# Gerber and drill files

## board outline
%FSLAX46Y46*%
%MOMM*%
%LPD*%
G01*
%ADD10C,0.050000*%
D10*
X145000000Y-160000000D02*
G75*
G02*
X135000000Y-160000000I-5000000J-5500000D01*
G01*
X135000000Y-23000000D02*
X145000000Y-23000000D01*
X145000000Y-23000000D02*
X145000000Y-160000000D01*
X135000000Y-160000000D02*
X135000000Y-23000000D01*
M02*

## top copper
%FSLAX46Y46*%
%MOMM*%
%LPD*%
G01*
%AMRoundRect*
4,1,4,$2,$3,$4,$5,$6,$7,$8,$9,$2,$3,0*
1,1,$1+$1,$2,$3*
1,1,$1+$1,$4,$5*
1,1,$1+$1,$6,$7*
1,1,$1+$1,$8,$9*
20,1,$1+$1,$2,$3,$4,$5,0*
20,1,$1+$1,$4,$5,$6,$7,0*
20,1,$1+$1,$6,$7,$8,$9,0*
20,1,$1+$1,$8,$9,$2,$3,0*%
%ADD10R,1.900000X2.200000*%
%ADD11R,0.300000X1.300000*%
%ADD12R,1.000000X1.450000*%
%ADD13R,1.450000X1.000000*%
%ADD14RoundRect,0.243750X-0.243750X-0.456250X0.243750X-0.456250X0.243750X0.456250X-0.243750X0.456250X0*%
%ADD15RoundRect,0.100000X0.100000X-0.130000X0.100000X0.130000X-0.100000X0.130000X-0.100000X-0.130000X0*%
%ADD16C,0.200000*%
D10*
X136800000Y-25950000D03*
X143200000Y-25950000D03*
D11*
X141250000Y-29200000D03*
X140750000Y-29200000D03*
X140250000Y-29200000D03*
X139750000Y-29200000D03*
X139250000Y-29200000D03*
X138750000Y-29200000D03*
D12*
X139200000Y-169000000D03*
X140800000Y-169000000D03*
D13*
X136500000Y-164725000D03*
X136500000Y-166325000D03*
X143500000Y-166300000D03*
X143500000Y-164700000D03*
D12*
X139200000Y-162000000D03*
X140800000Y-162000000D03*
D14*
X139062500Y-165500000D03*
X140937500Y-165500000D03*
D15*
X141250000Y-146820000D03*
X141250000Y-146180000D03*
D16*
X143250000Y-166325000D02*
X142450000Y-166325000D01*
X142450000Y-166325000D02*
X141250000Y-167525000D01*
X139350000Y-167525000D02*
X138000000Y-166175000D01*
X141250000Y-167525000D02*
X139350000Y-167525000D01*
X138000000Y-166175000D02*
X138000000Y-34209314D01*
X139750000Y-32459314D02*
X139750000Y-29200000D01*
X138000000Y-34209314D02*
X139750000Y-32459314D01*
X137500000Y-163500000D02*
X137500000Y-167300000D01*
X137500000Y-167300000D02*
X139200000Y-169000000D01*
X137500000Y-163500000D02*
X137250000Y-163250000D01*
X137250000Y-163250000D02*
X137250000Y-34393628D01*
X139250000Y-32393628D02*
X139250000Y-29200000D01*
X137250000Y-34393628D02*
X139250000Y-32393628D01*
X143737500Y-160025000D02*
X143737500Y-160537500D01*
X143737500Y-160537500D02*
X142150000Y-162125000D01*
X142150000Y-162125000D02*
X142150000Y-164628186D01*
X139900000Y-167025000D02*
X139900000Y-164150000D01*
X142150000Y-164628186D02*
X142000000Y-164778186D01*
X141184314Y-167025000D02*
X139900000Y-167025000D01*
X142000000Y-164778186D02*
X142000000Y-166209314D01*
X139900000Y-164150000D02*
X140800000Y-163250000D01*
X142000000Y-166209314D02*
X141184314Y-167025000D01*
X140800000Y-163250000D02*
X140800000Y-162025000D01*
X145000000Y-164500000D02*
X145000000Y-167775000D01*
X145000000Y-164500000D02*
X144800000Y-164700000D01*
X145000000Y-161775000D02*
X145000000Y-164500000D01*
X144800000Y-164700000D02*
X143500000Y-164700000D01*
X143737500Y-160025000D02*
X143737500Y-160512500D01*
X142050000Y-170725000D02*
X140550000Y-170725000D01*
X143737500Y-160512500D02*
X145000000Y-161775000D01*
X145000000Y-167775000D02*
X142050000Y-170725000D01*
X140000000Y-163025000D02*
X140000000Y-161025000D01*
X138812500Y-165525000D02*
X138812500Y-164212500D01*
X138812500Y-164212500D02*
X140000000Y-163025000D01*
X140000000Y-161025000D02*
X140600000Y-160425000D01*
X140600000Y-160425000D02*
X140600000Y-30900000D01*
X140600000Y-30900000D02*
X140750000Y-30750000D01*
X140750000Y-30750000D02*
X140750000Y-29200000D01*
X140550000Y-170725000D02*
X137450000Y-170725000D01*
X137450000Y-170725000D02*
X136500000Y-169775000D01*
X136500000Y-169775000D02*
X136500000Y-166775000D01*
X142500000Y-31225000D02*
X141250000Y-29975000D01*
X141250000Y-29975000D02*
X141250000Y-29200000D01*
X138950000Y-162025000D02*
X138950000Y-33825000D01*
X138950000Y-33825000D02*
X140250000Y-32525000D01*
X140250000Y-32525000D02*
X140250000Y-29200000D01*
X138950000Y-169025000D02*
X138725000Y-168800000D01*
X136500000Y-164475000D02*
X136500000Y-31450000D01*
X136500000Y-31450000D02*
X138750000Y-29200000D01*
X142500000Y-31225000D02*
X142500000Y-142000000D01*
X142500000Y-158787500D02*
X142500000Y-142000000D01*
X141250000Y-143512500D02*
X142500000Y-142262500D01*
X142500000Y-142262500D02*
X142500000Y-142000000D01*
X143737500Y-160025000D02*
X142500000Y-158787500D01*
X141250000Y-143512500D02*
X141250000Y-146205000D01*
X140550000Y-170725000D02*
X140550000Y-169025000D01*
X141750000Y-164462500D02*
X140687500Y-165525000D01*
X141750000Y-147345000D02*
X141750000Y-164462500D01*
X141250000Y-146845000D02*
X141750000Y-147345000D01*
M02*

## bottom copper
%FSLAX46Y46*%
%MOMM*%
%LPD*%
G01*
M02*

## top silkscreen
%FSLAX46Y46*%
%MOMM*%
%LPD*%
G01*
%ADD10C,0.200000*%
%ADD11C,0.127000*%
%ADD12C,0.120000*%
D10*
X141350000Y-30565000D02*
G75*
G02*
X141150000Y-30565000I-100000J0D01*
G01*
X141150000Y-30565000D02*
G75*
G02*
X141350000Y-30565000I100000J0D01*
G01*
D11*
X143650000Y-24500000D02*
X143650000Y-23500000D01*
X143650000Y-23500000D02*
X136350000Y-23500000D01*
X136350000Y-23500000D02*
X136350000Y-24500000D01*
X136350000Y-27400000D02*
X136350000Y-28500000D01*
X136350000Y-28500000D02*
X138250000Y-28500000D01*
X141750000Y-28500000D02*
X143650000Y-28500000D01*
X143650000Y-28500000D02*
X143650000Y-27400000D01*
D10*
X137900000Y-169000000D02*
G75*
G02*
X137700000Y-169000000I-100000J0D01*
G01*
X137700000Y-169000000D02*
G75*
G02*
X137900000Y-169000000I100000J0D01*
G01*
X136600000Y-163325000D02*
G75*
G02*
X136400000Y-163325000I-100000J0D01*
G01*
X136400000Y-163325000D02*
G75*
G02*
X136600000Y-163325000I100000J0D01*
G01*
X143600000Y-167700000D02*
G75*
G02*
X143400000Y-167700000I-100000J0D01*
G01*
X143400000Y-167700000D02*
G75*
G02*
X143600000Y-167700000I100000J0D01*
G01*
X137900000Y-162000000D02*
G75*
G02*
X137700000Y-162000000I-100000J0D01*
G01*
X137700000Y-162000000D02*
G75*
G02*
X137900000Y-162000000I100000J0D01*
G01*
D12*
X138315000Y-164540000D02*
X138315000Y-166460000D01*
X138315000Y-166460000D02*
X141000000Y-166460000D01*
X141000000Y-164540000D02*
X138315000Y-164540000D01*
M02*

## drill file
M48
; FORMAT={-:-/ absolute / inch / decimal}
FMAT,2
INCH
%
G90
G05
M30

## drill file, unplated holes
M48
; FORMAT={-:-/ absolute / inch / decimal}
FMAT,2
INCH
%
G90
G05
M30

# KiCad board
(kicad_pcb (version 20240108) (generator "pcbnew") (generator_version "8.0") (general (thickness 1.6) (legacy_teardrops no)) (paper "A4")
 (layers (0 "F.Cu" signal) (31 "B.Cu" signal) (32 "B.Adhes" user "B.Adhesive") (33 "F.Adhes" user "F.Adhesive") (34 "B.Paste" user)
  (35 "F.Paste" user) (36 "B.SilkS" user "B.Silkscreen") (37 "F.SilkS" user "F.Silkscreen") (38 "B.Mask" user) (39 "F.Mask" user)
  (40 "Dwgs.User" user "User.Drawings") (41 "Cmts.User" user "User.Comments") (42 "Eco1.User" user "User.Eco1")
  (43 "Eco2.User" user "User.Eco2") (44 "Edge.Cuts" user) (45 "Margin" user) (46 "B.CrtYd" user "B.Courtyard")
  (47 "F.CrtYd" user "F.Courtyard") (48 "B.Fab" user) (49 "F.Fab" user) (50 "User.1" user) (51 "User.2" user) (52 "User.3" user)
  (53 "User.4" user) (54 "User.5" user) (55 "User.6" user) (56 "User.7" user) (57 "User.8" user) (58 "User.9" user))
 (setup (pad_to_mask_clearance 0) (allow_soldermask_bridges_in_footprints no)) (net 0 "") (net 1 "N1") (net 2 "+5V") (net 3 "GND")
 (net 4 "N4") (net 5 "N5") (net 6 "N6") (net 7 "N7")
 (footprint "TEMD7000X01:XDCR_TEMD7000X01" (layer "F.Cu") (at 140 169)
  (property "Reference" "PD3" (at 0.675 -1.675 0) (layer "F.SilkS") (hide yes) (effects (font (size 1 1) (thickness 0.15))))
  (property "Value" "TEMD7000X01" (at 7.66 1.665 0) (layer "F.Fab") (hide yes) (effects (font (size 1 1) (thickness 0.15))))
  (fp_circle (center -2.2 0) (end -2.1 0) (stroke (width 0.2) (type solid)) (fill none) (layer "F.SilkS"))
  (pad "A" smd rect (at -0.8 0) (size 1 1.45) (layers "F.Cu" "F.Paste" "F.Mask") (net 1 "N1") (solder_mask_margin 0.102))
  (pad "C" smd rect (at 0.8 0) (size 1 1.45) (layers "F.Cu" "F.Paste" "F.Mask") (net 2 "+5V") (solder_mask_margin 0.102)))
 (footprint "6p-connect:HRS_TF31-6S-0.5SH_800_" (layer "F.Cu") (at 140 26)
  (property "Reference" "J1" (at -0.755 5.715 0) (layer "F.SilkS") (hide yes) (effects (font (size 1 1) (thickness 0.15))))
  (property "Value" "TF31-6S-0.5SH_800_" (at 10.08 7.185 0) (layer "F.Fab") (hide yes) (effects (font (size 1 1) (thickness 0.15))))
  (fp_line (start -3.65 -2.5) (end -3.65 -1.5) (stroke (width 0.127) (type solid)) (layer "F.SilkS"))
  (fp_line (start -3.65 1.4) (end -3.65 2.5) (stroke (width 0.127) (type solid)) (layer "F.SilkS"))
  (fp_line (start -3.65 2.5) (end -1.75 2.5) (stroke (width 0.127) (type solid)) (layer "F.SilkS"))
  (fp_line (start 1.75 2.5) (end 3.65 2.5) (stroke (width 0.127) (type solid)) (layer "F.SilkS"))
  (fp_line (start 3.65 -2.5) (end -3.65 -2.5) (stroke (width 0.127) (type solid)) (layer "F.SilkS"))
  (fp_line (start 3.65 -1.5) (end 3.65 -2.5) (stroke (width 0.127) (type solid)) (layer "F.SilkS"))
  (fp_line (start 3.65 2.5) (end 3.65 1.4) (stroke (width 0.127) (type solid)) (layer "F.SilkS"))
  (fp_circle (center 1.25 4.565) (end 1.35 4.565) (stroke (width 0.2) (type solid)) (fill none) (layer "F.SilkS"))
  (pad "1" smd rect (at 1.25 3.2) (size 0.3 1.3) (layers "F.Cu" "F.Paste" "F.Mask") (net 2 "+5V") (solder_mask_margin 0.02))
  (pad "2" smd rect (at 0.75 3.2) (size 0.3 1.3) (layers "F.Cu" "F.Paste" "F.Mask") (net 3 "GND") (solder_mask_margin 0.02))
  (pad "3" smd rect (at 0.25 3.2) (size 0.3 1.3) (layers "F.Cu" "F.Paste" "F.Mask") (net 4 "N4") (solder_mask_margin 0.02))
  (pad "4" smd rect (at -0.25 3.2) (size 0.3 1.3) (layers "F.Cu" "F.Paste" "F.Mask") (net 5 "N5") (solder_mask_margin 0.02))
  (pad "5" smd rect (at -0.75 3.2) (size 0.3 1.3) (layers "F.Cu" "F.Paste" "F.Mask") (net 1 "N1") (solder_mask_margin 0.02))
  (pad "6" smd rect (at -1.25 3.2) (size 0.3 1.3) (layers "F.Cu" "F.Paste" "F.Mask") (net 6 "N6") (solder_mask_margin 0.02))
  (pad "S1" smd rect (at -3.2 -0.05) (size 1.9 2.2) (layers "F.Cu" "F.Paste" "F.Mask") (solder_mask_margin 0.102))
  (pad "S2" smd rect (at 3.2 -0.05) (size 1.9 2.2) (layers "F.Cu" "F.Paste" "F.Mask") (solder_mask_margin 0.102)))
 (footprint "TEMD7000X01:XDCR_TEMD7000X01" (layer "F.Cu") (at 136.5 165.525 -90)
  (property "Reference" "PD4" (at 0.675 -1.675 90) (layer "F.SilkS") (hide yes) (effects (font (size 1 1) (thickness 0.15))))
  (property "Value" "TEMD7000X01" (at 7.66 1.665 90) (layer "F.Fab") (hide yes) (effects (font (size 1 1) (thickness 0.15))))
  (fp_circle (center -2.2 0) (end -2.1 0) (stroke (width 0.2) (type solid)) (fill none) (layer "F.SilkS"))
  (pad "A" smd rect (at -0.8 0 270) (size 1 1.45) (layers "F.Cu" "F.Paste" "F.Mask") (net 6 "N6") (solder_mask_margin 0.102))
  (pad "C" smd rect (at 0.8 0 270) (size 1 1.45) (layers "F.Cu" "F.Paste" "F.Mask") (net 2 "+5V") (solder_mask_margin 0.102)))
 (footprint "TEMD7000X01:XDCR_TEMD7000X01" (layer "F.Cu") (at 143.5 165.5 90)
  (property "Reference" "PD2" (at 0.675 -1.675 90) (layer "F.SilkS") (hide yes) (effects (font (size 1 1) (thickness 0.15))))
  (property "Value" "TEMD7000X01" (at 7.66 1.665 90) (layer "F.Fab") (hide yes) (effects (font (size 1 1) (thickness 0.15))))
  (fp_circle (center -2.2 0) (end -2.1 0) (stroke (width 0.2) (type solid)) (fill none) (layer "F.SilkS"))
  (pad "A" smd rect (at -0.8 0 90) (size 1 1.45) (layers "F.Cu" "F.Paste" "F.Mask") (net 5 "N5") (solder_mask_margin 0.102))
  (pad "C" smd rect (at 0.8 0 90) (size 1 1.45) (layers "F.Cu" "F.Paste" "F.Mask") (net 2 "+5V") (solder_mask_margin 0.102)))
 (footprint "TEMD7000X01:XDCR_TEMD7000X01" (layer "F.Cu") (at 140 162)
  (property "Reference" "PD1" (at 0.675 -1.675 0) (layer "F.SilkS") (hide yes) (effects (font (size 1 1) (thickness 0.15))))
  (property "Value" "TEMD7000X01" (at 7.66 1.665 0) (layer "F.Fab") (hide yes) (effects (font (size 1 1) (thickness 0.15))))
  (fp_circle (center -2.2 0) (end -2.1 0) (stroke (width 0.2) (type solid)) (fill none) (layer "F.SilkS"))
  (pad "A" smd rect (at -0.8 0) (size 1 1.45) (layers "F.Cu" "F.Paste" "F.Mask") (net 4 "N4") (solder_mask_margin 0.102))
  (pad "C" smd rect (at 0.8 0) (size 1 1.45) (layers "F.Cu" "F.Paste" "F.Mask") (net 2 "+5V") (solder_mask_margin 0.102)))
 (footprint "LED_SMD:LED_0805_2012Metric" (layer "F.Cu") (at 140 165.5)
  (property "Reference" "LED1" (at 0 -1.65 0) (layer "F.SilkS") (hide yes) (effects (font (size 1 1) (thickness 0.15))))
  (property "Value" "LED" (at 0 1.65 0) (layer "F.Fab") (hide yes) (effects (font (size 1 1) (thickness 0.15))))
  (fp_line (start -1.685 -0.96) (end -1.685 0.96) (stroke (width 0.12) (type solid)) (layer "F.SilkS"))
  (fp_line (start -1.685 0.96) (end 1 0.96) (stroke (width 0.12) (type solid)) (layer "F.SilkS"))
  (fp_line (start 1 -0.96) (end -1.685 -0.96) (stroke (width 0.12) (type solid)) (layer "F.SilkS"))
  (pad "1" smd roundrect (at -0.9375 0) (size 0.975 1.4) (layers "F.Cu" "F.Paste" "F.Mask") (roundrect_rratio 0.25) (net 3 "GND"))
  (pad "2" smd roundrect (at 0.9375 0) (size 0.975 1.4) (layers "F.Cu" "F.Paste" "F.Mask") (roundrect_rratio 0.25) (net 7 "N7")))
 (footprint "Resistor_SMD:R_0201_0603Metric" (layer "F.Cu") (at 141.25 146.5 90)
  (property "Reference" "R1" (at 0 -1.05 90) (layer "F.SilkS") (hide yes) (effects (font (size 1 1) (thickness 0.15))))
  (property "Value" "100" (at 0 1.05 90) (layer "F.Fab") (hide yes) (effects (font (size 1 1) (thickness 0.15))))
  (pad "" smd roundrect (at -0.345 0 90) (size 0.318 0.36) (layers "F.Paste") (roundrect_rratio 0.25))
  (pad "" smd roundrect (at 0.345 0 90) (size 0.318 0.36) (layers "F.Paste") (roundrect_rratio 0.25))
  (pad "1" smd roundrect (at -0.32 0 90) (size 0.46 0.4) (layers "F.Cu" "F.Mask") (roundrect_rratio 0.25) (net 7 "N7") (clearance 0.05))
  (pad "2" smd roundrect (at 0.32 0 90) (size 0.46 0.4) (layers "F.Cu" "F.Mask") (roundrect_rratio 0.25) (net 2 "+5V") (clearance 0.05)))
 (gr_line (start 135 23) (end 145 23) (stroke (width 0.05) (type default)) (layer "Edge.Cuts"))
 (gr_line (start 145 23) (end 145 160) (stroke (width 0.05) (type default)) (layer "Edge.Cuts"))
 (gr_line (start 135 160) (end 135 23) (stroke (width 0.05) (type default)) (layer "Edge.Cuts"))
 (gr_arc (start 145 160) (mid 140 172.933034) (end 135 160) (stroke (width 0.05) (type default)) (layer "Edge.Cuts"))
 (segment (start 143.7375 160.025) (end 143.7375 160.5375) (width 0.2) (layer "F.Cu") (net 2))
 (segment (start 144.8 164.7) (end 143.5 164.7) (width 0.2) (layer "F.Cu") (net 2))
 (segment (start 142 164.778186) (end 142 166.209314) (width 0.2) (layer "F.Cu") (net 2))
 (segment (start 145 164.5) (end 144.8 164.7) (width 0.2) (layer "F.Cu") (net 2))
 (segment (start 139.9 164.15) (end 140.8 163.25) (width 0.2) (layer "F.Cu") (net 2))
 (segment (start 140.55 170.725) (end 137.45 170.725) (width 0.2) (layer "F.Cu") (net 2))
 (segment (start 143.7375 160.025) (end 142.5 158.7875) (width 0.2) (layer "F.Cu") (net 2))
 (segment (start 139.9 167.025) (end 139.9 164.15) (width 0.2) (layer "F.Cu") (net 2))
 (segment (start 143.7375 160.5125) (end 145 161.775) (width 0.2) (layer "F.Cu") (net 2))
 (segment (start 140.8 163.25) (end 140.8 162.025) (width 0.2) (layer "F.Cu") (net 2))
 (segment (start 142.5 142.2625) (end 142.5 142) (width 0.2) (layer "F.Cu") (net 2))
 (segment (start 142.5 31.225) (end 142.5 142) (width 0.2) (layer "F.Cu") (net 2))
 (segment (start 141.25 29.975) (end 141.25 29.2) (width 0.2) (layer "F.Cu") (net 2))
 (segment (start 143.7375 160.025) (end 143.7375 160.5125) (width 0.2) (layer "F.Cu") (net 2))
 (segment (start 142.05 170.725) (end 140.55 170.725) (width 0.2) (layer "F.Cu") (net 2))
 (segment (start 142 166.209314) (end 141.184314 167.025) (width 0.2) (layer "F.Cu") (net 2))
 (segment (start 145 167.775) (end 142.05 170.725) (width 0.2) (layer "F.Cu") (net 2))
 (segment (start 142.15 164.628186) (end 142 164.778186) (width 0.2) (layer "F.Cu") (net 2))
 (segment (start 141.25 143.5125) (end 142.5 142.2625) (width 0.2) (layer "F.Cu") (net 2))
 (segment (start 142.5 158.7875) (end 142.5 142) (width 0.2) (layer "F.Cu") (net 2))
 (segment (start 145 161.775) (end 145 164.5) (width 0.2) (layer "F.Cu") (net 2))
 (segment (start 136.5 169.775) (end 136.5 166.775) (width 0.2) (layer "F.Cu") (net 2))
 (segment (start 141.184314 167.025) (end 139.9 167.025) (width 0.2) (layer "F.Cu") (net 2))
 (segment (start 141.25 143.5125) (end 141.25 146.205) (width 0.2) (layer "F.Cu") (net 2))
 (segment (start 145 164.5) (end 145 167.775) (width 0.2) (layer "F.Cu") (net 2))
 (segment (start 142.5 31.225) (end 141.25 29.975) (width 0.2) (layer "F.Cu") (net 2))
 (segment (start 140.55 170.725) (end 140.55 169.025) (width 0.2) (layer "F.Cu") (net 2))
 (segment (start 143.7375 160.5375) (end 142.15 162.125) (width 0.2) (layer "F.Cu") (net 2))
 (segment (start 142.15 162.125) (end 142.15 164.628186) (width 0.2) (layer "F.Cu") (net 2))
 (segment (start 137.45 170.725) (end 136.5 169.775) (width 0.2) (layer "F.Cu") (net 2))
 (segment (start 140.6 160.425) (end 140.6 30.9) (width 0.2) (layer "F.Cu") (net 3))
 (segment (start 140.6 30.9) (end 140.75 30.75) (width 0.2) (layer "F.Cu") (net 3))
 (segment (start 138.8125 165.525) (end 138.8125 164.2125) (width 0.2) (layer "F.Cu") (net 3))
 (segment (start 140 161.025) (end 140.6 160.425) (width 0.2) (layer "F.Cu") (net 3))
 (segment (start 140.75 30.75) (end 140.75 29.2) (width 0.2) (layer "F.Cu") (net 3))
 (segment (start 140 163.025) (end 140 161.025) (width 0.2) (layer "F.Cu") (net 3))
 (segment (start 138.8125 164.2125) (end 140 163.025) (width 0.2) (layer "F.Cu") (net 3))
 (segment (start 141.75 164.4625) (end 140.6875 165.525) (width 0.2) (layer "F.Cu") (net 7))
 (segment (start 141.75 147.345) (end 141.75 164.4625) (width 0.2) (layer "F.Cu") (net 7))
 (segment (start 141.25 146.845) (end 141.75 147.345) (width 0.2) (layer "F.Cu") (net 7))
 (segment (start 140.25 32.525) (end 140.25 29.2) (width 0.2) (layer "F.Cu") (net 4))
 (segment (start 138.95 33.825) (end 140.25 32.525) (width 0.2) (layer "F.Cu") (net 4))
 (segment (start 138.95 162.025) (end 138.95 33.825) (width 0.2) (layer "F.Cu") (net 4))
 (segment (start 136.5 164.475) (end 136.5 31.45) (width 0.2) (layer "F.Cu") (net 6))
 (segment (start 136.5 31.45) (end 138.75 29.2) (width 0.2) (layer "F.Cu") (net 6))
 (segment (start 139.25 32.393628) (end 139.25 29.2) (width 0.2) (layer "F.Cu") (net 1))
 (segment (start 138.95 169.025) (end 138.725 168.8) (width 0.2) (layer "F.Cu") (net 1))
 (segment (start 137.5 163.5) (end 137.25 163.25) (width 0.2) (layer "F.Cu") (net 1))
 (segment (start 137.5 163.5) (end 137.5 167.3) (width 0.2) (layer "F.Cu") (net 1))
 (segment (start 137.5 167.3) (end 139.2 169) (width 0.2) (layer "F.Cu") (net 1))
 (segment (start 137.25 163.25) (end 137.25 34.393628) (width 0.2) (layer "F.Cu") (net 1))
 (segment (start 137.25 34.393628) (end 139.25 32.393628) (width 0.2) (layer "F.Cu") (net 1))
 (segment (start 142.45 166.325) (end 141.25 167.525) (width 0.2) (layer "F.Cu") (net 5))
 (segment (start 138 166.175) (end 138 34.209314) (width 0.2) (layer "F.Cu") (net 5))
 (segment (start 138 34.209314) (end 139.75 32.459314) (width 0.2) (layer "F.Cu") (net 5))
 (segment (start 141.25 167.525) (end 139.35 167.525) (width 0.2) (layer "F.Cu") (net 5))
 (segment (start 139.75 32.459314) (end 139.75 29.2) (width 0.2) (layer "F.Cu") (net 5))
 (segment (start 143.25 166.325) (end 142.45 166.325) (width 0.2) (layer "F.Cu") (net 5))
 (segment (start 139.35 167.525) (end 138 166.175) (width 0.2) (layer "F.Cu") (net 5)))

